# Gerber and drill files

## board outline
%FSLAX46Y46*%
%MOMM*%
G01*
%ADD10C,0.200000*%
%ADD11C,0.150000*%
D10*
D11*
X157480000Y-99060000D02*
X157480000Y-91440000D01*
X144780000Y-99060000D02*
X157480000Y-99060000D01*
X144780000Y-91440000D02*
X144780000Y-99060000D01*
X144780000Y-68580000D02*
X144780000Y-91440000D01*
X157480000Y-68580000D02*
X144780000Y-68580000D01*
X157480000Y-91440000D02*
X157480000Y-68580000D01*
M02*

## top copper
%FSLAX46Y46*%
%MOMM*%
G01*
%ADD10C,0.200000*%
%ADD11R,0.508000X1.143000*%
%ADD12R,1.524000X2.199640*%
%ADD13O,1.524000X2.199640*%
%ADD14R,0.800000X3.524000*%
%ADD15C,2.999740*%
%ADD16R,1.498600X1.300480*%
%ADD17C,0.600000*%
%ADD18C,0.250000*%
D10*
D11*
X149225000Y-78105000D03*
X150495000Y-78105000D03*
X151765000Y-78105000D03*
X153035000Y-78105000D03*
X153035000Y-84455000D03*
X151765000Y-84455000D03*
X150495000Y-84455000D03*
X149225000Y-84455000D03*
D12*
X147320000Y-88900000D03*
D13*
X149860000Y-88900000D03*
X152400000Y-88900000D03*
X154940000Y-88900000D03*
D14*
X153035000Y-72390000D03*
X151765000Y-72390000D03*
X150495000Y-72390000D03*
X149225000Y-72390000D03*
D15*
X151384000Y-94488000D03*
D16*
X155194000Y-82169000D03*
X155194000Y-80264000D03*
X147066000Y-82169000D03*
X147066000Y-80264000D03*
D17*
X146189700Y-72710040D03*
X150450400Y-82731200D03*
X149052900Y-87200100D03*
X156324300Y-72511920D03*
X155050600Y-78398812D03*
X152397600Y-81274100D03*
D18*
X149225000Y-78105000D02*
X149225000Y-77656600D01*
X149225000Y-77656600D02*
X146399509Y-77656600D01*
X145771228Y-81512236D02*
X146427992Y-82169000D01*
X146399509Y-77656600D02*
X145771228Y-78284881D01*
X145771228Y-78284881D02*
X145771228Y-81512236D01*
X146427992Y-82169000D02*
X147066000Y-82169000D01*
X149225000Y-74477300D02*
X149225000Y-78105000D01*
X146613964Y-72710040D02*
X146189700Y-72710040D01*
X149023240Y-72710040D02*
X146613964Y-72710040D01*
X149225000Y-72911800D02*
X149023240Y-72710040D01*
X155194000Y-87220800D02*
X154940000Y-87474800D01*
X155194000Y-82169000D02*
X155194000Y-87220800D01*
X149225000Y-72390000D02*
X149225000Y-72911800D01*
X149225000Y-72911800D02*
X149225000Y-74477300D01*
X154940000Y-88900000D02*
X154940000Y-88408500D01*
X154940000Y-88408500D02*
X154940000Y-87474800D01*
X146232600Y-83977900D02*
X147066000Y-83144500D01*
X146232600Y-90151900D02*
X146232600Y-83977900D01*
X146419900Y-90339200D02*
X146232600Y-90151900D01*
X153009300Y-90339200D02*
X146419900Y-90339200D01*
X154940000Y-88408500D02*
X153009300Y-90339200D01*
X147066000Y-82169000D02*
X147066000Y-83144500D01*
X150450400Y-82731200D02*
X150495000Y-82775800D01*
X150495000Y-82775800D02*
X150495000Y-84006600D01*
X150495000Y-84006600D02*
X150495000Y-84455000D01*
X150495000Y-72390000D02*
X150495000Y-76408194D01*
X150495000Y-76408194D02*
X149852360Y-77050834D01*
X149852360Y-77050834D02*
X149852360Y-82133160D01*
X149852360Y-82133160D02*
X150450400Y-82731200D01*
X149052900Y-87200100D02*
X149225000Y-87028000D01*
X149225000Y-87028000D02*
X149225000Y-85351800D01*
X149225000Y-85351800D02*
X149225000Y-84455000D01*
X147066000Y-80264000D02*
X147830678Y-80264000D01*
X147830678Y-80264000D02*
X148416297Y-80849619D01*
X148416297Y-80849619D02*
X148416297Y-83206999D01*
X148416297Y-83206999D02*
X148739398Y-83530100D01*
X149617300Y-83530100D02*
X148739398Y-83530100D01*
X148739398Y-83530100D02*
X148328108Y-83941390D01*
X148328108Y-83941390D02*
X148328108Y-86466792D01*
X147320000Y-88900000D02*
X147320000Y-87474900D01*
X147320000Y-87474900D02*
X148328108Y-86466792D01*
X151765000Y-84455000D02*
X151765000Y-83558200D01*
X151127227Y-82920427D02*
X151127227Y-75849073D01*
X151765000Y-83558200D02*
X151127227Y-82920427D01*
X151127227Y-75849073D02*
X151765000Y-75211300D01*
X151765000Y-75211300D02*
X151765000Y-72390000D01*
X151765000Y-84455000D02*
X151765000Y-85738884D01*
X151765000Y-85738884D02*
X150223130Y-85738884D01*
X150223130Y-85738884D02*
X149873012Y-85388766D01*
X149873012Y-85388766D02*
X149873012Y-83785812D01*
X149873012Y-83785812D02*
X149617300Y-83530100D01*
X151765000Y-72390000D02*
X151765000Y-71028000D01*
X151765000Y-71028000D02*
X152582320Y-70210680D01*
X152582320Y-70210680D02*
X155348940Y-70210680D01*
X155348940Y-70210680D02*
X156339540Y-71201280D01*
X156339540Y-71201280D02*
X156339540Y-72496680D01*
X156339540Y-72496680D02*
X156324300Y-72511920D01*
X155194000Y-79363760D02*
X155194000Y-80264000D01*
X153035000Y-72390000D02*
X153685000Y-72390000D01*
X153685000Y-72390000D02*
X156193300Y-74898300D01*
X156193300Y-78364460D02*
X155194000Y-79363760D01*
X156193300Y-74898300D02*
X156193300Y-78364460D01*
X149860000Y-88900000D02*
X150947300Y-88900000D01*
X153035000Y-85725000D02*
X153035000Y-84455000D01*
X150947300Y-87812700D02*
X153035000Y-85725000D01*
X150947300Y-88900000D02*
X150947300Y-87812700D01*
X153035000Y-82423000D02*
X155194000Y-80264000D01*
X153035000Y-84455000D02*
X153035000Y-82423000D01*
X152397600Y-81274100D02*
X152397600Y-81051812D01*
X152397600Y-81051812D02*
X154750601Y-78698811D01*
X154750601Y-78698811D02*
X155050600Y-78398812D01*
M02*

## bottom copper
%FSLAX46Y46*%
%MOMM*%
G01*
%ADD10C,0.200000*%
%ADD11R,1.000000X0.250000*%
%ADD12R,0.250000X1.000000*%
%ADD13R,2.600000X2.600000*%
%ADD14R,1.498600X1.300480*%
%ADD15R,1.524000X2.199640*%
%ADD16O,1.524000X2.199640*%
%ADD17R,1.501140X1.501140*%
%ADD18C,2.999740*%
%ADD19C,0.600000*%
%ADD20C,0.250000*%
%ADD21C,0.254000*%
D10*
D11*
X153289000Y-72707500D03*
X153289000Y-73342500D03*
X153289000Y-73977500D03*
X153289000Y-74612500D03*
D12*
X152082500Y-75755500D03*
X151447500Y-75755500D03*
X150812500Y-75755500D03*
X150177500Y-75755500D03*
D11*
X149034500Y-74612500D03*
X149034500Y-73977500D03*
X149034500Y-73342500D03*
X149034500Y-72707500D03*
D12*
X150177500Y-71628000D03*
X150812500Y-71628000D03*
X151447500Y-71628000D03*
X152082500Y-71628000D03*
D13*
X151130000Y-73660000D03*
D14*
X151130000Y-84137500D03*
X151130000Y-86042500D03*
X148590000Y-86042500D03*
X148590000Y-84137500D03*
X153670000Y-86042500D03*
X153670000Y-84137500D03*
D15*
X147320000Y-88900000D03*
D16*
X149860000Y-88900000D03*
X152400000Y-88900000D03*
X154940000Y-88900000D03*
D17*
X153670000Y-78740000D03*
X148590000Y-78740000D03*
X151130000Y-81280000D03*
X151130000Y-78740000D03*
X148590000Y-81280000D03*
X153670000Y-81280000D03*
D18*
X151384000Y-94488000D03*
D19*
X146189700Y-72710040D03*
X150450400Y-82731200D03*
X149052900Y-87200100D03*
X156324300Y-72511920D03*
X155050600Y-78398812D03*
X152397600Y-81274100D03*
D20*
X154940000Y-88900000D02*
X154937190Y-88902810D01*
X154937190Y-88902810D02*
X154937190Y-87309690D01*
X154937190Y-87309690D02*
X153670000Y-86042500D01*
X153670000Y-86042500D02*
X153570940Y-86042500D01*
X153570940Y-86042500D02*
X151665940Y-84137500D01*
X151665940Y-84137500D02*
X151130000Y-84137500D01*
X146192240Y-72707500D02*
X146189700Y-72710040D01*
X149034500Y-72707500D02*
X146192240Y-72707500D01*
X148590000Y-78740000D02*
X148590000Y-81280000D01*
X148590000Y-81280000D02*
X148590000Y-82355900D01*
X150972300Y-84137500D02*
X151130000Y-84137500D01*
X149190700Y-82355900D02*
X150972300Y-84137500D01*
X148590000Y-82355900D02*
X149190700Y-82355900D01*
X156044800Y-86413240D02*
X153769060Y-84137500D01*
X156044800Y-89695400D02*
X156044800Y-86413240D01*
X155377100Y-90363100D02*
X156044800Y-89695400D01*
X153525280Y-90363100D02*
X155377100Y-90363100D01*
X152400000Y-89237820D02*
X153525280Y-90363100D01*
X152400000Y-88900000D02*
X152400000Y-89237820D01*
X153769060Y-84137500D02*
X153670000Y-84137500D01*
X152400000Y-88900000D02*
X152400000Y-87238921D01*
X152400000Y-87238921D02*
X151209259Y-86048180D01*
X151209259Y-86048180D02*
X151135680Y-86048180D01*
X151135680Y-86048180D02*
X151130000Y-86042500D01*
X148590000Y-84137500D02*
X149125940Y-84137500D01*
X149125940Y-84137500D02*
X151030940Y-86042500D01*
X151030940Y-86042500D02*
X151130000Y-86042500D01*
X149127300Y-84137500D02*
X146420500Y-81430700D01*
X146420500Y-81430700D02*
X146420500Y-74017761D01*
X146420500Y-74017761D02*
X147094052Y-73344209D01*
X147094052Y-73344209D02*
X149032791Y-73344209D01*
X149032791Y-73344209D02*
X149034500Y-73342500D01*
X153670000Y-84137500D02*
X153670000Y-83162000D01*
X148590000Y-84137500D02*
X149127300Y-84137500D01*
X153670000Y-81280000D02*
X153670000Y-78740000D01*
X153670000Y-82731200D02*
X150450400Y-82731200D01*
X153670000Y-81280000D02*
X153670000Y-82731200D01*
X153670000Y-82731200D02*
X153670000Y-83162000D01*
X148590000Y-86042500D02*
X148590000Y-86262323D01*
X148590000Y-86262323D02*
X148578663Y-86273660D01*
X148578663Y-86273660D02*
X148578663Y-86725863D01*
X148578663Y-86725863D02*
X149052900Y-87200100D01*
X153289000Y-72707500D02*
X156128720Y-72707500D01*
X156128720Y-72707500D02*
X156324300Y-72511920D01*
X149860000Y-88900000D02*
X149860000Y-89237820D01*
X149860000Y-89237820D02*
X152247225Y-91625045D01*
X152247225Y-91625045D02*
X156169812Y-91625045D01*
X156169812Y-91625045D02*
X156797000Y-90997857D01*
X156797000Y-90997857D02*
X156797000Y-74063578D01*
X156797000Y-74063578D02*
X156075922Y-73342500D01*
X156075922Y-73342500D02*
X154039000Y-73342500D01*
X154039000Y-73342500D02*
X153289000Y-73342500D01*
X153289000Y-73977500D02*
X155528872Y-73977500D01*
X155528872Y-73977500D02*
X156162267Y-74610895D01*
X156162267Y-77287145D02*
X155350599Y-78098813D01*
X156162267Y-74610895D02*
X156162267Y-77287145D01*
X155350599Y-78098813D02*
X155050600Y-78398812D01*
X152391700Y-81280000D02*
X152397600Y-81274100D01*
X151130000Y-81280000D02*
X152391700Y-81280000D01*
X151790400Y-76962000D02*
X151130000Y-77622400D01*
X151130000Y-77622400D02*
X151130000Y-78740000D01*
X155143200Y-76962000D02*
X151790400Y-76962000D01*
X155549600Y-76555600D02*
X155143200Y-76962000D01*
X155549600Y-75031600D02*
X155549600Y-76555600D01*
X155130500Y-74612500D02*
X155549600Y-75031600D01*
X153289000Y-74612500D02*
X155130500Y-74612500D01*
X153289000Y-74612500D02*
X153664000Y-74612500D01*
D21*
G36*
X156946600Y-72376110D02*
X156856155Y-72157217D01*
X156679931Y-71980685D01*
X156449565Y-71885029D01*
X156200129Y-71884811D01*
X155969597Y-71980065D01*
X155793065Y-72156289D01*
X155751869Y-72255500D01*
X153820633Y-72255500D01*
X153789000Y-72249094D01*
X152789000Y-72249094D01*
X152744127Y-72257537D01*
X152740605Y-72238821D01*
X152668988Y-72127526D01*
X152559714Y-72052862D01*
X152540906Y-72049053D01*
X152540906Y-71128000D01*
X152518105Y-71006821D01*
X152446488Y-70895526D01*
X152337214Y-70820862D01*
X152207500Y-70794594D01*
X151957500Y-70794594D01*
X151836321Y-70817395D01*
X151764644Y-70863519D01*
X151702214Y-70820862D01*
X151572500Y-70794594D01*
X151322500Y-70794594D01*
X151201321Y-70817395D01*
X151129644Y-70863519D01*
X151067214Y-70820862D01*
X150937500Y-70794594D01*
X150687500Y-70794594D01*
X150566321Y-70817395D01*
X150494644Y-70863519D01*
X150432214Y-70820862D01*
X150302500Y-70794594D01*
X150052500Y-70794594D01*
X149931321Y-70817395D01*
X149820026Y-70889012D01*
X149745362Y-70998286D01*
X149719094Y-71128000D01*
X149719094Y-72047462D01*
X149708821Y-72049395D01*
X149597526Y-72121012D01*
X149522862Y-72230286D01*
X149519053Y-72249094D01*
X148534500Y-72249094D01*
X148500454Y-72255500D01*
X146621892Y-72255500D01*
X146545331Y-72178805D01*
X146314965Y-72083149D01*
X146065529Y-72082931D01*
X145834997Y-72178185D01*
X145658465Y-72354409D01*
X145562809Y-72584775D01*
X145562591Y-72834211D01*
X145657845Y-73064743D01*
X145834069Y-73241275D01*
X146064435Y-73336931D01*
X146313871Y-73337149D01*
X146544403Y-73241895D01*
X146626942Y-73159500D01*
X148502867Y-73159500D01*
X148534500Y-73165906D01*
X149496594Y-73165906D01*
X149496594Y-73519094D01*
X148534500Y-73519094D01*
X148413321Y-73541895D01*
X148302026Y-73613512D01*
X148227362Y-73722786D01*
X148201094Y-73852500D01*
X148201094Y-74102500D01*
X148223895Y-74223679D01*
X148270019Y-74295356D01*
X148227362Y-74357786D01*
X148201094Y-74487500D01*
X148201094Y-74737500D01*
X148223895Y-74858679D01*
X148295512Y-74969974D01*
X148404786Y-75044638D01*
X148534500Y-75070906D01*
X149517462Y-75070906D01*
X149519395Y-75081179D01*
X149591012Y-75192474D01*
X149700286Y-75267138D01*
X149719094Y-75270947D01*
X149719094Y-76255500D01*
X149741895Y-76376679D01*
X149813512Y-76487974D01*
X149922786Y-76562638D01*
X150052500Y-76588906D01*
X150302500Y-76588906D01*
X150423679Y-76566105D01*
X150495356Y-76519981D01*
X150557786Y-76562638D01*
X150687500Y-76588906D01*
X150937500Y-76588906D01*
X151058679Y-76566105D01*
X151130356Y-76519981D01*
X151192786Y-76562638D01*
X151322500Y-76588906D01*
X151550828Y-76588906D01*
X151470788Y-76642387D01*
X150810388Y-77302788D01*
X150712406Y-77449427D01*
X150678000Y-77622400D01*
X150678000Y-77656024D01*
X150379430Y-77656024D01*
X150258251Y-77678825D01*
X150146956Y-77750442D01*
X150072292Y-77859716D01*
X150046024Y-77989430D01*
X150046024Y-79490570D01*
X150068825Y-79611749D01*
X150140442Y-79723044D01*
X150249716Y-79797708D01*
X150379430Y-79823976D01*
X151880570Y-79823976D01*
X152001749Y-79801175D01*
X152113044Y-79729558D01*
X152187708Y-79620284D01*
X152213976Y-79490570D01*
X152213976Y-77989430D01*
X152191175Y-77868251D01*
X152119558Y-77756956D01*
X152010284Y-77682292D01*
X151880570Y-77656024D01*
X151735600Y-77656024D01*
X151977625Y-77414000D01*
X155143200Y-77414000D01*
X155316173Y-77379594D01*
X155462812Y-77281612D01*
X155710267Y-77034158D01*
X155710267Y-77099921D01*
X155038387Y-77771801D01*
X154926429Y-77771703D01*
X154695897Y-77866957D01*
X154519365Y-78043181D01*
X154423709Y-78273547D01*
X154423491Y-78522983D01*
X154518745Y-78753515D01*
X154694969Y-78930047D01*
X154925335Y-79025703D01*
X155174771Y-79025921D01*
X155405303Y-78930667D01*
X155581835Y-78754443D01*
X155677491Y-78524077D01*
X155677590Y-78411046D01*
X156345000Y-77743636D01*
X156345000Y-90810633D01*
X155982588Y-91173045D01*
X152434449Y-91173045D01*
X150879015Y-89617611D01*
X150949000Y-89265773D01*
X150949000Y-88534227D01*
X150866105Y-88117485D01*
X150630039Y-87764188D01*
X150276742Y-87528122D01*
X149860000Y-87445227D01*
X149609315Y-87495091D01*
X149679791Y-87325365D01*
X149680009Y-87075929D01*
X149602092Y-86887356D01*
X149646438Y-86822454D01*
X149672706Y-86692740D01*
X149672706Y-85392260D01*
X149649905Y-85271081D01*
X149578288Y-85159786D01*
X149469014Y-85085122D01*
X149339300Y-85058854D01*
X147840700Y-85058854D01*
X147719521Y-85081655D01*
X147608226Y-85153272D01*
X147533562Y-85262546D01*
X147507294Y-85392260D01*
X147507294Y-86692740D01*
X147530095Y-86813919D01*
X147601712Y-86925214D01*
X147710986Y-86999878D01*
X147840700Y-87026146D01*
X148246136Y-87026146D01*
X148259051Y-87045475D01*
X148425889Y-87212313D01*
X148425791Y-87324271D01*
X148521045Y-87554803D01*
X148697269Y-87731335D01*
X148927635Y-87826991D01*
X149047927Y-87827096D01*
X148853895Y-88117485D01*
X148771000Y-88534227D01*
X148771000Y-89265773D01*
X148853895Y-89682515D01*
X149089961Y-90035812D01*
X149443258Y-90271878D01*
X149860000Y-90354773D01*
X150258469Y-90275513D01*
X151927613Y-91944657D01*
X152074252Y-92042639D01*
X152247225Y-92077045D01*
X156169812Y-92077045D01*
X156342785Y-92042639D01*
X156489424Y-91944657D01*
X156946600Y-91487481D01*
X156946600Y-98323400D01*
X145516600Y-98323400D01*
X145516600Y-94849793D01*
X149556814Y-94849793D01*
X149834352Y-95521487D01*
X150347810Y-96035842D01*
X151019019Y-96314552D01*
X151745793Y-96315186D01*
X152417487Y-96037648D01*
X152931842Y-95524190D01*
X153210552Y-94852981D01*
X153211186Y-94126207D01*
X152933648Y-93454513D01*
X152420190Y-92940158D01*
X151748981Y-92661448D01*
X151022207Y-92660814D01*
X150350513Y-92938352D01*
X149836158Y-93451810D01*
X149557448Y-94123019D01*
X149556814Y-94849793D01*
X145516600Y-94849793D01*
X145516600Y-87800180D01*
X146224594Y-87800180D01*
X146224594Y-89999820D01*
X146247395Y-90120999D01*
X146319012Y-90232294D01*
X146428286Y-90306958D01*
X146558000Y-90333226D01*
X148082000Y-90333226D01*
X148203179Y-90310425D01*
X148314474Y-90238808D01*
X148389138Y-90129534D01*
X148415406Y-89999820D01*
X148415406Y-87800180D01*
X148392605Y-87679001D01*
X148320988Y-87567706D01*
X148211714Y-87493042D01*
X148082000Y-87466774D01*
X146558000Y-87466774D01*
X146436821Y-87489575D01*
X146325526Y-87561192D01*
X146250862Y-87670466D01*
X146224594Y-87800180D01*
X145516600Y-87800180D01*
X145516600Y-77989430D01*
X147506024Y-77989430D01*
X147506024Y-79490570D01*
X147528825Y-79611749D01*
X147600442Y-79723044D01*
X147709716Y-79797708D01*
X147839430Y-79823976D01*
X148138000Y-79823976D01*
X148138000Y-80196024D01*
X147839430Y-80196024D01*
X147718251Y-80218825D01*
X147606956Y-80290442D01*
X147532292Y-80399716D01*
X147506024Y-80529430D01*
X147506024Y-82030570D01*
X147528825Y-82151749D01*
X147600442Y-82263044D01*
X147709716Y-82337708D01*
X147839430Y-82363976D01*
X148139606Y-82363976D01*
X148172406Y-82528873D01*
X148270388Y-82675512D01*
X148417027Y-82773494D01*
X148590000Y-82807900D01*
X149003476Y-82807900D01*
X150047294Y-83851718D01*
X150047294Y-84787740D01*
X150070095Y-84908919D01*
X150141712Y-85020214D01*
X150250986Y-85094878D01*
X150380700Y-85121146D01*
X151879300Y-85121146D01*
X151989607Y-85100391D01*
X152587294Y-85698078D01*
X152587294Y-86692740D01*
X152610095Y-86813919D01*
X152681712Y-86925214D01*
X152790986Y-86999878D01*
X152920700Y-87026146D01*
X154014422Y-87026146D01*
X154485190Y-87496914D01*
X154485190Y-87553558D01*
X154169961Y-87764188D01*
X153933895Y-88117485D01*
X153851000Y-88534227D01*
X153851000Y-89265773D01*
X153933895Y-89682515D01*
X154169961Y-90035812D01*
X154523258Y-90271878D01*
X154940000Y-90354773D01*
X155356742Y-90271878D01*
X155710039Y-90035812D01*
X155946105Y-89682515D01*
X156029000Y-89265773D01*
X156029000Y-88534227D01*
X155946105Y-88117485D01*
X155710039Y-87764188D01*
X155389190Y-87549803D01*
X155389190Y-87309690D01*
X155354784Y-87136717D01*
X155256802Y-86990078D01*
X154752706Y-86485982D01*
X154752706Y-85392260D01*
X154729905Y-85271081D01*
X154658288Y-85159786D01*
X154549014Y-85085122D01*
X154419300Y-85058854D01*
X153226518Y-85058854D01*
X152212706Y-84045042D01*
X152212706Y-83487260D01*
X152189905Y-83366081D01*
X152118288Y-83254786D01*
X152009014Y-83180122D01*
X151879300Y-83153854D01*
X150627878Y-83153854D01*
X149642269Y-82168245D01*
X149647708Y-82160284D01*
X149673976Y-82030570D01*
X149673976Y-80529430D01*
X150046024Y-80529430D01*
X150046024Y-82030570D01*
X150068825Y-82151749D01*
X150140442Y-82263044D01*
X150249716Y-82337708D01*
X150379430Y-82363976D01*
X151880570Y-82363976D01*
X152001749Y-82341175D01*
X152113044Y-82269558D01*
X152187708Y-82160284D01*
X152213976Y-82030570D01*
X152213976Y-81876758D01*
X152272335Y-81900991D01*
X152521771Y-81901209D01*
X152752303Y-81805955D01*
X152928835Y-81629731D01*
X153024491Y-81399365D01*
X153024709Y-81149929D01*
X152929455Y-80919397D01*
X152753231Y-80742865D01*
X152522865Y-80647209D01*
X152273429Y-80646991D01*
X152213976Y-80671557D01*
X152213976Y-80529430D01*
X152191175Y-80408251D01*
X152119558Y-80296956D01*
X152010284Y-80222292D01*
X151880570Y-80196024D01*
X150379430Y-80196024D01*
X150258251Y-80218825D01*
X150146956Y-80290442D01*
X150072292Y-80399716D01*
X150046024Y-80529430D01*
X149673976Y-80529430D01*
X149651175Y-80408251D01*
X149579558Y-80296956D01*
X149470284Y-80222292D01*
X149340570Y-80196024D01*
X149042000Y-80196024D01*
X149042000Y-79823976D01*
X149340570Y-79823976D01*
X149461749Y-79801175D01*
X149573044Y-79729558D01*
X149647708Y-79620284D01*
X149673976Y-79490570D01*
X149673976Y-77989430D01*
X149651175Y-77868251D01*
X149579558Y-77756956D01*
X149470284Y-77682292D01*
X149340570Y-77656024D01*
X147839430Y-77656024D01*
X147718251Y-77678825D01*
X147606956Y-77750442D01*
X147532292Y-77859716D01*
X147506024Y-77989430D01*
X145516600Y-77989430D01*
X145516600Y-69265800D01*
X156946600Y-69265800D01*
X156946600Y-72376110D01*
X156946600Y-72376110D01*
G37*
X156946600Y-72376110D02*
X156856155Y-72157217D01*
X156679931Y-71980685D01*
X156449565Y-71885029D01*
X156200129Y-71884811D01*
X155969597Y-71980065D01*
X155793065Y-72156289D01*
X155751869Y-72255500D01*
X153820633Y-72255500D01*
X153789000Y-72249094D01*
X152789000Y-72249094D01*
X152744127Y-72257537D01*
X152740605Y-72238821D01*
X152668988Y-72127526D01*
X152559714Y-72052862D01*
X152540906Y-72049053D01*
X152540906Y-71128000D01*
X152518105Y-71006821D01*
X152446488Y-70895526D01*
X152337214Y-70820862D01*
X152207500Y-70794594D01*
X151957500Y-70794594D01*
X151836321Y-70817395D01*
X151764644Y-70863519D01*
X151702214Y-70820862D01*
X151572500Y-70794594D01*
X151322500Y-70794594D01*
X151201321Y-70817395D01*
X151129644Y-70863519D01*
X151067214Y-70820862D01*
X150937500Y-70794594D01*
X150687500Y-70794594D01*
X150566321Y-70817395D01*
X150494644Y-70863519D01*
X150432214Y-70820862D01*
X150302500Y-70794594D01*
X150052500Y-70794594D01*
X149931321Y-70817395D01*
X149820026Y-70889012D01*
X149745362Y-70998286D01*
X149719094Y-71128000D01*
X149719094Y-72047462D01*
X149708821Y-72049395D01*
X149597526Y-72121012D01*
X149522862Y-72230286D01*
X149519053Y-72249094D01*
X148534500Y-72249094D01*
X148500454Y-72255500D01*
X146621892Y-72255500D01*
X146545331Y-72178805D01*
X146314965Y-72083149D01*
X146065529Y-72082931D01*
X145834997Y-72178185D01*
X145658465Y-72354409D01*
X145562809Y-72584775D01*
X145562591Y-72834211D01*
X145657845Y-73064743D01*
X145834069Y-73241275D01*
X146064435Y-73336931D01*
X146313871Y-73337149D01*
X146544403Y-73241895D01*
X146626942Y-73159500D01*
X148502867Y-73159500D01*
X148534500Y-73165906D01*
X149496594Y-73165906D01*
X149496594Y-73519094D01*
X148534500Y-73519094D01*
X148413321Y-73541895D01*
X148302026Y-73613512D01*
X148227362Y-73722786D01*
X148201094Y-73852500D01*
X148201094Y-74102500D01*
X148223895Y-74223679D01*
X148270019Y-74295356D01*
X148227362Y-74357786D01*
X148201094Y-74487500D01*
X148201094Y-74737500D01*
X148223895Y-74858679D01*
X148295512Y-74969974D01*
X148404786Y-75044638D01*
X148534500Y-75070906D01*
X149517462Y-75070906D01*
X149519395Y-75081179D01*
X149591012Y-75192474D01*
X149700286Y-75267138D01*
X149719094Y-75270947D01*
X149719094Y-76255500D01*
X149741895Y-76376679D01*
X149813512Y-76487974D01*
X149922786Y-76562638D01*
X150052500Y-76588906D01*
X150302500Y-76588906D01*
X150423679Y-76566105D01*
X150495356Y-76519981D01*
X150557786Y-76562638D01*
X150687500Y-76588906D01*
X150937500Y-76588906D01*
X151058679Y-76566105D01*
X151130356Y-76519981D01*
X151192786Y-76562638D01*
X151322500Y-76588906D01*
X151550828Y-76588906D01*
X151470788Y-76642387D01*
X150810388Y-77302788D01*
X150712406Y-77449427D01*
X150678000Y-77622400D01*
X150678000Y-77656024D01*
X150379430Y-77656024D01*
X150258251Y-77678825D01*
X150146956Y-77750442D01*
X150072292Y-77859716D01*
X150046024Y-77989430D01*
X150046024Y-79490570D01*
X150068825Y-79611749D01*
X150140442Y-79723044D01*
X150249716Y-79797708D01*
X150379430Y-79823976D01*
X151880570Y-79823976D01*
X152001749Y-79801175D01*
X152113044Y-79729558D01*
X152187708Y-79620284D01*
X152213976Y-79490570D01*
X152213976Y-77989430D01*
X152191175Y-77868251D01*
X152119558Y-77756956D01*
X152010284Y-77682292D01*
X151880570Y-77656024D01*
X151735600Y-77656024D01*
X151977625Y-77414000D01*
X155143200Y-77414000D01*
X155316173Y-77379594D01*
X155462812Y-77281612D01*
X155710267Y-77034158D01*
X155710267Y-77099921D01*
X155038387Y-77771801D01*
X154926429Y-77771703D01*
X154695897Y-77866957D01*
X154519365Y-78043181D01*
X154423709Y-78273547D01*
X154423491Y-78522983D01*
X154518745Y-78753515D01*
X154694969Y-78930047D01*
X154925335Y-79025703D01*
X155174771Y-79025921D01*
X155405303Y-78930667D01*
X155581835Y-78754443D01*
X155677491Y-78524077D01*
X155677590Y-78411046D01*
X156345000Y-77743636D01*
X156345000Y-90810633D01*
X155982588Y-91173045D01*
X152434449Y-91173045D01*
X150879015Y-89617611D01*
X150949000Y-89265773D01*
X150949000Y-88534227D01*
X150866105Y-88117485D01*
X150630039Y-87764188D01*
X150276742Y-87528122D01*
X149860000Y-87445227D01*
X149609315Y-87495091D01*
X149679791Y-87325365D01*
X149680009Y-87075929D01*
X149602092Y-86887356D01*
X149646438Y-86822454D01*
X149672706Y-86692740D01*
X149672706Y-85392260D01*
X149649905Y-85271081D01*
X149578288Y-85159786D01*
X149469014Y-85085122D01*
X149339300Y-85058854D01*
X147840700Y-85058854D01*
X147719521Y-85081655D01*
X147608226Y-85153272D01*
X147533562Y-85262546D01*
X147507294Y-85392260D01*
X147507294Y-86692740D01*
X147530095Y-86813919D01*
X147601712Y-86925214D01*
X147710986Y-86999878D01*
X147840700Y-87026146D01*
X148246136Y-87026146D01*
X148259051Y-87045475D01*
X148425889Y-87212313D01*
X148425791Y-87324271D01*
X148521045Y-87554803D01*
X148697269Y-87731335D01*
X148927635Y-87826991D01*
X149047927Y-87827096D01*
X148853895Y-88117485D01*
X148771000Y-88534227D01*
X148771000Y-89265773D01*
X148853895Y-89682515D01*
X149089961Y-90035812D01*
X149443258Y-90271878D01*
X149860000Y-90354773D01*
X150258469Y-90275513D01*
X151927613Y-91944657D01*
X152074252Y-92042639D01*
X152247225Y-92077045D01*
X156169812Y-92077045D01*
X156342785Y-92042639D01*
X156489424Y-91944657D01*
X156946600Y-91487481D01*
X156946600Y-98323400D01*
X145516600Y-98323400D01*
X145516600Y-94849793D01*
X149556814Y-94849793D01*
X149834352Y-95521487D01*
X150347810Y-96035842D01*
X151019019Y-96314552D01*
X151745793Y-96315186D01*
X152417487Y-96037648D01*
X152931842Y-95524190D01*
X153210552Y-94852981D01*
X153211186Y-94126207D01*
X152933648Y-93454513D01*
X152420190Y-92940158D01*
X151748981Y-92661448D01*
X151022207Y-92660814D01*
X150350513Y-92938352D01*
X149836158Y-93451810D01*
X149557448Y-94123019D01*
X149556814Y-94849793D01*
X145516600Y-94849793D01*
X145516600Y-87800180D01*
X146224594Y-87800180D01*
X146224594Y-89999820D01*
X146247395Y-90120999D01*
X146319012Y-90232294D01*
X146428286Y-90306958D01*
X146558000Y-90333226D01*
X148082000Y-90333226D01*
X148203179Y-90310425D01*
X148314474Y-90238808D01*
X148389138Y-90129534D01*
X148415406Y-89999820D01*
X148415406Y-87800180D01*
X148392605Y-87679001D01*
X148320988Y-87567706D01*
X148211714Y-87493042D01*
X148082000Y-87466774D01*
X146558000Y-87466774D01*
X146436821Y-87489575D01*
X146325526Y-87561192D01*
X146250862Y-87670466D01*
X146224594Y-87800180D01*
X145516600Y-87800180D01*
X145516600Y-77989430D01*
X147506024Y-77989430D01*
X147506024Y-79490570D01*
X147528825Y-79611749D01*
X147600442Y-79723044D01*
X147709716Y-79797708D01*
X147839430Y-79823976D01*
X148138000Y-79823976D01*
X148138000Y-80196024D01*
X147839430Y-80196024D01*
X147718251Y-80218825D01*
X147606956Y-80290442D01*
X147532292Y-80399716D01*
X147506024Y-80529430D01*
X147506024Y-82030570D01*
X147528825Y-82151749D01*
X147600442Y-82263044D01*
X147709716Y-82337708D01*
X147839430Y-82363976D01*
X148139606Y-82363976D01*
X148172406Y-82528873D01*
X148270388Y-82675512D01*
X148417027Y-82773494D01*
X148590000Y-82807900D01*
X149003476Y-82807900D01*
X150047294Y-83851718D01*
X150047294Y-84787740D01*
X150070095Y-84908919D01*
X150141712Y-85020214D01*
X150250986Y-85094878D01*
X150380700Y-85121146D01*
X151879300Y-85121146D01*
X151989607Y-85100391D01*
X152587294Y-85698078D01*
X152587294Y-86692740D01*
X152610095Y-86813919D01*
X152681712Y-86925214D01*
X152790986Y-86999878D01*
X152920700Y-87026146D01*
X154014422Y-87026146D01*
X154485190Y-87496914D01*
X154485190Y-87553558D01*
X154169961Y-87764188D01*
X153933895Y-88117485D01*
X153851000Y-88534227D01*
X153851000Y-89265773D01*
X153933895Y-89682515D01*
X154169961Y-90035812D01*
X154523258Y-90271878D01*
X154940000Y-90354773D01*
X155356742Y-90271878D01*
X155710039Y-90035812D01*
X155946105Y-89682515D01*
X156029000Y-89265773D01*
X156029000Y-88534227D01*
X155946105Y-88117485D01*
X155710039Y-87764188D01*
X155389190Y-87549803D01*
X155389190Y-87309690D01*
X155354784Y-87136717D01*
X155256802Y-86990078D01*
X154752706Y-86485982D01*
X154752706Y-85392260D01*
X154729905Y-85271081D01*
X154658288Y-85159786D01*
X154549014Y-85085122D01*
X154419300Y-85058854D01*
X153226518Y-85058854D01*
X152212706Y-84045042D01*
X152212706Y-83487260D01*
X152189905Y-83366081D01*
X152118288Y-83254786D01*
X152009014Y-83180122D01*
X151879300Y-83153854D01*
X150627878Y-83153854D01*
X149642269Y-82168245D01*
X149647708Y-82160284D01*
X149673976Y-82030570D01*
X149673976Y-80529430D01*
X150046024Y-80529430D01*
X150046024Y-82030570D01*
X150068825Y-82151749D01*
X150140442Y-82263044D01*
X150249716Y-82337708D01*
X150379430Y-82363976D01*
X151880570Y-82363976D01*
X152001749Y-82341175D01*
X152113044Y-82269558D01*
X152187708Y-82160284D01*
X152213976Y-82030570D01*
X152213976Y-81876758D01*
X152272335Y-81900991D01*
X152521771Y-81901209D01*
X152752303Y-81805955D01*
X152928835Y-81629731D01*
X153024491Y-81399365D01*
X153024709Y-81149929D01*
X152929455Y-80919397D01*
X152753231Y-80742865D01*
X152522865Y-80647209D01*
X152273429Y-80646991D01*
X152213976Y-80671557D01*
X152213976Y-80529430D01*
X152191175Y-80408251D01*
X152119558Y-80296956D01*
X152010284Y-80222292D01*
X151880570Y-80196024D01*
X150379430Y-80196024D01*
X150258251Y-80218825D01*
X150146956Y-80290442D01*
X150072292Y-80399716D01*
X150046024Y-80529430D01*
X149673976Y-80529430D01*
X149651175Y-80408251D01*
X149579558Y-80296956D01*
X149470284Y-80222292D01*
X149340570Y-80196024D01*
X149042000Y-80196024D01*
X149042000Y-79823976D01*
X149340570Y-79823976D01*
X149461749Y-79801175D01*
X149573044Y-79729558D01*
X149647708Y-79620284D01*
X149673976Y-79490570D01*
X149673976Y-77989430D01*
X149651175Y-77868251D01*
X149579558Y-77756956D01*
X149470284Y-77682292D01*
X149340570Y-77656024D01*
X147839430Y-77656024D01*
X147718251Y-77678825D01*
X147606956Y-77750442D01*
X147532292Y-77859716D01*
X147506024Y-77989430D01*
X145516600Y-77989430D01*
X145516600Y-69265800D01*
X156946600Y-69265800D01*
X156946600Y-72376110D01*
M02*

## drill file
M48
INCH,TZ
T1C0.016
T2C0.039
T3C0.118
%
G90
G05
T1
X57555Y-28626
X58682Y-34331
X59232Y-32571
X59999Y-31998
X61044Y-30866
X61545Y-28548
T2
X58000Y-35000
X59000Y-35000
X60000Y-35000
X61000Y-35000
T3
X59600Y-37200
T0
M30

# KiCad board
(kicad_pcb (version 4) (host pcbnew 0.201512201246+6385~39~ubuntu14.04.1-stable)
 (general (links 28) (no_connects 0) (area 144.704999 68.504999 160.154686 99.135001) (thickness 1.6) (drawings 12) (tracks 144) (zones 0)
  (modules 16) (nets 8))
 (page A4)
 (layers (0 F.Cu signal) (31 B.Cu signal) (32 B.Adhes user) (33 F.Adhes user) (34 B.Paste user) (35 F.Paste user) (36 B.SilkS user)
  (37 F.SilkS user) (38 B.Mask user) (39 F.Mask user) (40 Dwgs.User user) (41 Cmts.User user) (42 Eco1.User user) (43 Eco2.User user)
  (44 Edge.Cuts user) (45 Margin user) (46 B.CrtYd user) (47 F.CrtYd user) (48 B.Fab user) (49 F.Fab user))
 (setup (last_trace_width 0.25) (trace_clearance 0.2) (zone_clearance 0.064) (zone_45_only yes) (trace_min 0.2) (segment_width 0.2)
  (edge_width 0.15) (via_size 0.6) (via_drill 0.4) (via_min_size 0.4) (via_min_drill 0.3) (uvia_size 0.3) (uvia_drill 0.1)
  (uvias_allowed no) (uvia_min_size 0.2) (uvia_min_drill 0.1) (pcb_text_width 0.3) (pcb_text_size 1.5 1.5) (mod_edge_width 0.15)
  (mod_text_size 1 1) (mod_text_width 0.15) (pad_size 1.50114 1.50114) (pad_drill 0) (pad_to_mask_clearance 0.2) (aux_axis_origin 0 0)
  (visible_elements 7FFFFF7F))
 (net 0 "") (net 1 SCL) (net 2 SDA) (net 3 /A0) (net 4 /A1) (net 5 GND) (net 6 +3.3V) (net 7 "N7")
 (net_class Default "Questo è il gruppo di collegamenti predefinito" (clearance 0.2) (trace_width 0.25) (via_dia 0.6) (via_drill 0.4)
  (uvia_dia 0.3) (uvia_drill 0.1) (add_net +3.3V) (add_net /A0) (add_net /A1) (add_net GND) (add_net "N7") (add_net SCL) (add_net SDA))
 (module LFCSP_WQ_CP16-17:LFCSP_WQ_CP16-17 (layer B.Cu) (at 151.13 73.66 180)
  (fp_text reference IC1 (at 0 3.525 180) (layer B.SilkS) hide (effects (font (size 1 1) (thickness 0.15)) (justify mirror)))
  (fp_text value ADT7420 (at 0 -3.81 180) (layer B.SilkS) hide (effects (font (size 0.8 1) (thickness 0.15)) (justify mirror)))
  (pad 1 smd rect (at -2.159 0.9525 180) (size 1 0.25) (layers B.Cu B.Paste B.Mask) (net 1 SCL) (solder_mask_margin 0.07))
  (pad 2 smd rect (at -2.159 0.3175 180) (size 1 0.25) (layers B.Cu B.Paste B.Mask) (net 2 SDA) (solder_mask_margin 0.07))
  (pad 3 smd rect (at -2.159 -0.3175 180) (size 1 0.25) (layers B.Cu B.Paste B.Mask) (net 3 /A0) (solder_mask_margin 0.07))
  (pad 4 smd rect (at -2.159 -0.9525 180) (size 1 0.25) (layers B.Cu B.Paste B.Mask) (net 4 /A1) (solder_mask_margin 0.07))
  (pad 5 smd rect (at -0.9525 -2.0955 90) (size 1 0.25) (layers B.Cu B.Paste B.Mask) (solder_mask_margin 0.07))
  (pad 6 smd rect (at -0.3175 -2.0955 90) (size 1 0.25) (layers B.Cu B.Paste B.Mask) (solder_mask_margin 0.07))
  (pad 7 smd rect (at 0.3175 -2.0955 90) (size 1 0.25) (layers B.Cu B.Paste B.Mask) (solder_mask_margin 0.07))
  (pad 8 smd rect (at 0.9525 -2.0955 90) (size 1 0.25) (layers B.Cu B.Paste B.Mask) (solder_mask_margin 0.07))
  (pad 9 smd rect (at 2.0955 -0.9525 270) (size 0.25 1) (layers B.Cu B.Paste B.Mask) (solder_mask_margin 0.07))
  (pad 10 smd rect (at 2.0955 -0.3175 270) (size 0.25 1) (layers B.Cu B.Paste B.Mask) (solder_mask_margin 0.07))
  (pad 11 smd rect (at 2.0955 0.3175 270) (size 0.25 1) (layers B.Cu B.Paste B.Mask) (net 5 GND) (solder_mask_margin 0.07))
  (pad 12 smd rect (at 2.0955 0.9525 270) (size 0.25 1) (layers B.Cu B.Paste B.Mask) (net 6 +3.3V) (solder_mask_margin 0.07))
  (pad 13 smd rect (at 0.9525 2.032 180) (size 0.25 1) (layers B.Cu B.Paste B.Mask) (solder_mask_margin 0.07))
  (pad 14 smd rect (at 0.3175 2.032 180) (size 0.25 1) (layers B.Cu B.Paste B.Mask) (solder_mask_margin 0.07))
  (pad 15 smd rect (at -0.3175 2.032 180) (size 0.25 1) (layers B.Cu B.Paste B.Mask) (solder_mask_margin 0.07))
  (pad 16 smd rect (at -0.9525 2.032 180) (size 0.25 1) (layers B.Cu B.Paste B.Mask) (solder_mask_margin 0.07))
  (pad 17 smd rect (at 0 0 180) (size 2.6 2.6) (layers B.Cu B.Paste B.Mask)))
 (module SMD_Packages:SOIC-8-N (layer F.Cu) (at 151.13 81.28)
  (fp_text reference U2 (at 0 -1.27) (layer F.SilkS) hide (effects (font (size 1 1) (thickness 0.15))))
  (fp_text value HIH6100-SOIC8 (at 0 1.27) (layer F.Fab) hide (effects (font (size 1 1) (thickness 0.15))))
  (pad 8 smd rect (at -1.905 -3.175) (size 0.508 1.143) (layers F.Cu F.Paste F.Mask) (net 6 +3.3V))
  (pad 7 smd rect (at -0.635 -3.175) (size 0.508 1.143) (layers F.Cu F.Paste F.Mask))
  (pad 6 smd rect (at 0.635 -3.175) (size 0.508 1.143) (layers F.Cu F.Paste F.Mask))
  (pad 5 smd rect (at 1.905 -3.175) (size 0.508 1.143) (layers F.Cu F.Paste F.Mask))
  (pad 4 smd rect (at 1.905 3.175) (size 0.508 1.143) (layers F.Cu F.Paste F.Mask) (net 2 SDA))
  (pad 3 smd rect (at 0.635 3.175) (size 0.508 1.143) (layers F.Cu F.Paste F.Mask) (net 1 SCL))
  (pad 2 smd rect (at -0.635 3.175) (size 0.508 1.143) (layers F.Cu F.Paste F.Mask) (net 5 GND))
  (pad 1 smd rect (at -1.905 3.175) (size 0.508 1.143) (layers F.Cu F.Paste F.Mask) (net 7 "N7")))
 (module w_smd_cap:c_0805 (layer B.Cu) (at 151.13 85.09 90)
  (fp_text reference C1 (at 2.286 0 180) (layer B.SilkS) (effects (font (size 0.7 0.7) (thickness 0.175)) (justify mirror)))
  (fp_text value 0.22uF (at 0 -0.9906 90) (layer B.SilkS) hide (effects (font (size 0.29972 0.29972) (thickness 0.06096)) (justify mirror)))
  (pad 1 smd rect (at 0.9525 0 90) (size 1.30048 1.4986) (layers B.Cu B.Paste B.Mask) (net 6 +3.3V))
  (pad 2 smd rect (at -0.9525 0 90) (size 1.30048 1.4986) (layers B.Cu B.Paste B.Mask) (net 5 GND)))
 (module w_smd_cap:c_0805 (layer B.Cu) (at 148.59 85.09 270)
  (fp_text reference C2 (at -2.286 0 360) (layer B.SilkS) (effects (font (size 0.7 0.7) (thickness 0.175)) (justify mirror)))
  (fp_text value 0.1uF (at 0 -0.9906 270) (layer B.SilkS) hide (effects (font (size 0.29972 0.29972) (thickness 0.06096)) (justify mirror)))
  (pad 1 smd rect (at 0.9525 0 270) (size 1.30048 1.4986) (layers B.Cu B.Paste B.Mask) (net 7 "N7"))
  (pad 2 smd rect (at -0.9525 0 270) (size 1.30048 1.4986) (layers B.Cu B.Paste B.Mask) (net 5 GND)))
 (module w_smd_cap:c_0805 (layer B.Cu) (at 153.67 85.09 270)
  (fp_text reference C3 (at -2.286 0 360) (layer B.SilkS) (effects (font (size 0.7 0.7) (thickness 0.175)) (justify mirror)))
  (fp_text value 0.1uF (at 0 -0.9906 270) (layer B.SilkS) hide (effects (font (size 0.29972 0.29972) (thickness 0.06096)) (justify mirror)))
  (pad 1 smd rect (at 0.9525 0 270) (size 1.30048 1.4986) (layers B.Cu B.Paste B.Mask) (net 6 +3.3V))
  (pad 2 smd rect (at -0.9525 0 270) (size 1.30048 1.4986) (layers B.Cu B.Paste B.Mask) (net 5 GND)))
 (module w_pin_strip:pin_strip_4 (layer F.Cu) (at 151.13 88.9)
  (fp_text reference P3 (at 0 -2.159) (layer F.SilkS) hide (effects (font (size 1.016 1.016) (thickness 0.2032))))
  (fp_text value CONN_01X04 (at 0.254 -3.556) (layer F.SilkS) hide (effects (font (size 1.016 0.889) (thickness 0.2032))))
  (pad 1 thru_hole rect (at -3.81 0) (size 1.524 2.19964) (drill 1.00076) (layers *.Cu *.Mask F.SilkS) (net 1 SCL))
  (pad 2 thru_hole oval (at -1.27 0) (size 1.524 2.19964) (drill 1.00076) (layers *.Cu *.Mask F.SilkS) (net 2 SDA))
  (pad 3 thru_hole oval (at 1.27 0) (size 1.524 2.19964) (drill 1.00076) (layers *.Cu *.Mask F.SilkS) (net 5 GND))
  (pad 4 thru_hole oval (at 3.81 0) (size 1.524 2.19964) (drill 1.00076) (layers *.Cu *.Mask F.SilkS) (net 6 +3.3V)))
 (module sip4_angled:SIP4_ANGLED (layer F.Cu) (at 151.13 71.12)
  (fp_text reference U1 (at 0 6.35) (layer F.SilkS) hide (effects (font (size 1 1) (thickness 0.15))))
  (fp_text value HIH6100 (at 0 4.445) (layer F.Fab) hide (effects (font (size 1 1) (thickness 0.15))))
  (pad 4 smd rect (at 1.905 1.27) (size 0.8 3.524) (layers F.Cu F.Paste F.Mask) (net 2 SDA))
  (pad 3 smd rect (at 0.635 1.27) (size 0.8 3.524) (layers F.Cu F.Paste F.Mask) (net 1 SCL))
  (pad 2 smd rect (at -0.635 1.27) (size 0.8 3.524) (layers F.Cu F.Paste F.Mask) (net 5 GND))
  (pad 1 smd rect (at -1.905 1.27) (size 0.8 3.524) (layers F.Cu F.Paste F.Mask) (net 6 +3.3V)))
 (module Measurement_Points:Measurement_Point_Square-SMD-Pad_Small (layer B.Cu) (at 153.67 78.74)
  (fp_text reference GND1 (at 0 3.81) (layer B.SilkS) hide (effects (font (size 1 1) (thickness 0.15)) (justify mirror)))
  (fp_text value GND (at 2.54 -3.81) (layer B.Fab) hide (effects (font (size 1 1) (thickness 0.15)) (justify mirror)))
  (pad 1 smd rect (at 0 0) (size 1.50114 1.50114) (layers B.Cu B.Paste B.Mask) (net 5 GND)))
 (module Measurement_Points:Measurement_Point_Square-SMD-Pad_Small (layer B.Cu) (at 148.59 78.74)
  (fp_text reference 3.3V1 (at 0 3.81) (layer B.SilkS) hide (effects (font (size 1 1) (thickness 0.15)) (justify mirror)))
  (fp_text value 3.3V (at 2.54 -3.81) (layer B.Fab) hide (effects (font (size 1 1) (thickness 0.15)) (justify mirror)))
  (pad 1 smd rect (at 0 0) (size 1.50114 1.50114) (layers B.Cu B.Paste B.Mask) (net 6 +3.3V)))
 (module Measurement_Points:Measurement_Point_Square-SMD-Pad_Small (layer B.Cu) (at 151.13 81.28)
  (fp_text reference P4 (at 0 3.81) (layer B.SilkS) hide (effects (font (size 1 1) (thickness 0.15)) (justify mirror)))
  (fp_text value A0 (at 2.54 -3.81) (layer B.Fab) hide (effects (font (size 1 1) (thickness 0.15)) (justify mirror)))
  (pad 1 smd rect (at 0 0) (size 1.50114 1.50114) (layers B.Cu B.Paste B.Mask) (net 3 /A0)))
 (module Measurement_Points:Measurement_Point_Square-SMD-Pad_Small (layer B.Cu) (at 151.13 78.74)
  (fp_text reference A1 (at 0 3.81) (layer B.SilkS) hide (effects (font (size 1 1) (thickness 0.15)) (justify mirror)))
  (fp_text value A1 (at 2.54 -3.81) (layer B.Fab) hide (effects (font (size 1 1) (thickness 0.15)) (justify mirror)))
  (pad 1 smd rect (at 0 0) (size 1.50114 1.50114) (layers B.Cu B.Paste B.Mask) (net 4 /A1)))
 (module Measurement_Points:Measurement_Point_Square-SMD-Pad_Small (layer F.Cu) (at 148.59 81.28)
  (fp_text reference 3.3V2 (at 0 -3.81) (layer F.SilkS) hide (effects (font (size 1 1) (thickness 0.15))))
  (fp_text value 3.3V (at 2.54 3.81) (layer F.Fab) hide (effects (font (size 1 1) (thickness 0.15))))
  (pad 1 smd rect (at 0 0) (size 1.50114 1.50114) (layers B.Cu B.Paste B.Mask) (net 6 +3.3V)))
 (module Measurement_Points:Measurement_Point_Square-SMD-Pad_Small (layer F.Cu) (at 153.67 81.28)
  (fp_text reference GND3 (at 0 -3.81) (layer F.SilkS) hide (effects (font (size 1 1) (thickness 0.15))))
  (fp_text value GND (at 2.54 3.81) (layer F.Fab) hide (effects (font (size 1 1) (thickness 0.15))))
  (pad 1 smd rect (at 0 0) (size 1.50114 1.50114) (layers B.Cu B.Paste B.Mask) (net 5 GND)))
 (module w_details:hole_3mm (layer F.Cu) (at 151.384 94.488)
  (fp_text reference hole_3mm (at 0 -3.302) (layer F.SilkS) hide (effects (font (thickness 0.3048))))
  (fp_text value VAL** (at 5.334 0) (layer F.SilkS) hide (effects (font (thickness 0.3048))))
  (pad 1 thru_hole circle (at 0 0) (size 2.99974 2.99974) (drill 2.99974) (layers *.Cu F.SilkS)))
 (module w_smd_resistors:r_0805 (layer F.Cu) (at 155.194 81.2165 270)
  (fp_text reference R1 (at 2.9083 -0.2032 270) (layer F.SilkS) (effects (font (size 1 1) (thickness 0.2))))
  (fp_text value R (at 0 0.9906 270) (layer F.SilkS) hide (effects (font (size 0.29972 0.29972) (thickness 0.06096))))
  (pad 1 smd rect (at 0.9525 0 270) (size 1.30048 1.4986) (layers F.Cu F.Paste F.Mask) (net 6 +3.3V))
  (pad 2 smd rect (at -0.9525 0 270) (size 1.30048 1.4986) (layers F.Cu F.Paste F.Mask) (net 2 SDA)))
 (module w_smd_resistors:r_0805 (layer F.Cu) (at 147.066 81.2165 270)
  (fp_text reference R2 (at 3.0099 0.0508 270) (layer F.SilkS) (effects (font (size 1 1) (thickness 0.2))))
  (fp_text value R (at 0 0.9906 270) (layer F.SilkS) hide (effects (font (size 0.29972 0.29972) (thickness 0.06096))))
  (pad 1 smd rect (at 0.9525 0 270) (size 1.30048 1.4986) (layers F.Cu F.Paste F.Mask) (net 6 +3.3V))
  (pad 2 smd rect (at -0.9525 0 270) (size 1.30048 1.4986) (layers F.Cu F.Paste F.Mask) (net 1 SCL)))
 (gr_line (start 157.48 99.06) (end 157.48 91.44) (angle 90) (layer Edge.Cuts) (width 0.15))
 (gr_line (start 144.78 99.06) (end 157.48 99.06) (angle 90) (layer Edge.Cuts) (width 0.15))
 (gr_line (start 144.78 91.44) (end 144.78 99.06) (angle 90) (layer Edge.Cuts) (width 0.15))
 (gr_line (start 144.78 68.58) (end 144.78 91.44) (angle 90) (layer Edge.Cuts) (width 0.15))
 (gr_line (start 157.48 68.58) (end 144.78 68.58) (angle 90) (layer Edge.Cuts) (width 0.15))
 (gr_line (start 157.48 91.44) (end 157.48 68.58) (angle 90) (layer Edge.Cuts) (width 0.15))
 (segment (start 154.94 88.9) (end 154.93719 88.90281) (width 0.25) (layer B.Cu) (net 6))
 (segment (start 154.93719 88.90281) (end 154.93719 87.30969) (width 0.25) (layer B.Cu) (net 6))
 (segment (start 154.93719 87.30969) (end 153.67 86.0425) (width 0.25) (layer B.Cu) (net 6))
 (segment (start 149.225 78.105) (end 149.225 77.6566) (width 0.25) (layer F.Cu) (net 6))
 (segment (start 149.225 77.6566) (end 146.399509 77.6566) (width 0.25) (layer F.Cu) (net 6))
 (segment (start 145.771228 81.512236) (end 146.427992 82.169) (width 0.25) (layer F.Cu) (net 6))
 (segment (start 146.399509 77.6566) (end 145.771228 78.284881) (width 0.25) (layer F.Cu) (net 6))
 (segment (start 145.771228 78.284881) (end 145.771228 81.512236) (width 0.25) (layer F.Cu) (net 6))
 (segment (start 146.427992 82.169) (end 147.066 82.169) (width 0.25) (layer F.Cu) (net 6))
 (segment (start 149.225 74.4773) (end 149.225 78.105) (width 0.25) (layer F.Cu) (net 6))
 (segment (start 153.67 86.0425) (end 153.57094 86.0425) (width 0.25) (layer B.Cu) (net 6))
 (segment (start 153.57094 86.0425) (end 151.66594 84.1375) (width 0.25) (layer B.Cu) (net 6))
 (segment (start 151.66594 84.1375) (end 151.13 84.1375) (width 0.25) (layer B.Cu) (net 6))
 (segment (start 146.613964 72.71004) (end 146.1897 72.71004) (width 0.25) (layer F.Cu) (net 6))
 (segment (start 149.02324 72.71004) (end 146.613964 72.71004) (width 0.25) (layer F.Cu) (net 6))
 (segment (start 149.225 72.9118) (end 149.02324 72.71004) (width 0.25) (layer F.Cu) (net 6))
 (segment (start 146.19224 72.7075) (end 146.1897 72.71004) (width 0.25) (layer B.Cu) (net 6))
 (segment (start 149.0345 72.7075) (end 146.19224 72.7075) (width 0.25) (layer B.Cu) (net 6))
 (via (at 146.1897 72.71004) (size 0.6) (drill 0.4) (layers F.Cu B.Cu) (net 6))
 (segment (start 155.194 87.2208) (end 154.94 87.4748) (width 0.25) (layer F.Cu) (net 6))
 (segment (start 155.194 82.169) (end 155.194 87.2208) (width 0.25) (layer F.Cu) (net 6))
 (segment (start 149.225 72.39) (end 149.225 72.9118) (width 0.25) (layer F.Cu) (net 6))
 (segment (start 149.225 72.9118) (end 149.225 74.4773) (width 0.25) (layer F.Cu) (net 6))
 (segment (start 148.59 78.74) (end 148.59 81.28) (width 0.25) (layer B.Cu) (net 6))
 (segment (start 148.59 81.28) (end 148.59 82.3559) (width 0.25) (layer B.Cu) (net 6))
 (segment (start 150.9723 84.1375) (end 151.13 84.1375) (width 0.25) (layer B.Cu) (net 6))
 (segment (start 149.1907 82.3559) (end 150.9723 84.1375) (width 0.25) (layer B.Cu) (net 6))
 (segment (start 148.59 82.3559) (end 149.1907 82.3559) (width 0.25) (layer B.Cu) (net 6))
 (segment (start 154.94 88.9) (end 154.94 88.4085) (width 0.25) (layer F.Cu) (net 6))
 (segment (start 154.94 88.4085) (end 154.94 87.4748) (width 0.25) (layer F.Cu) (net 6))
 (segment (start 146.2326 83.9779) (end 147.066 83.1445) (width 0.25) (layer F.Cu) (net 6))
 (segment (start 146.2326 90.1519) (end 146.2326 83.9779) (width 0.25) (layer F.Cu) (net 6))
 (segment (start 146.4199 90.3392) (end 146.2326 90.1519) (width 0.25) (layer F.Cu) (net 6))
 (segment (start 153.0093 90.3392) (end 146.4199 90.3392) (width 0.25) (layer F.Cu) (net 6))
 (segment (start 154.94 88.4085) (end 153.0093 90.3392) (width 0.25) (layer F.Cu) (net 6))
 (segment (start 147.066 82.169) (end 147.066 83.1445) (width 0.25) (layer F.Cu) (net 6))
 (segment (start 150.4504 82.7312) (end 150.495 82.7758) (width 0.25) (layer F.Cu) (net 5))
 (segment (start 150.495 82.7758) (end 150.495 84.0066) (width 0.25) (layer F.Cu) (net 5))
 (segment (start 150.495 84.0066) (end 150.495 84.455) (width 0.25) (layer F.Cu) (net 5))
 (segment (start 156.0448 86.41324) (end 153.76906 84.1375) (width 0.25) (layer B.Cu) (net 5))
 (segment (start 156.0448 89.6954) (end 156.0448 86.41324) (width 0.25) (layer B.Cu) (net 5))
 (segment (start 155.3771 90.3631) (end 156.0448 89.6954) (width 0.25) (layer B.Cu) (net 5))
 (segment (start 153.52528 90.3631) (end 155.3771 90.3631) (width 0.25) (layer B.Cu) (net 5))
 (segment (start 152.4 89.23782) (end 153.52528 90.3631) (width 0.25) (layer B.Cu) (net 5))
 (segment (start 152.4 88.9) (end 152.4 89.23782) (width 0.25) (layer B.Cu) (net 5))
 (segment (start 153.76906 84.1375) (end 153.67 84.1375) (width 0.25) (layer B.Cu) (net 5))
 (segment (start 152.4 88.9) (end 152.4 87.238921) (width 0.25) (layer B.Cu) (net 5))
 (segment (start 152.4 87.238921) (end 151.209259 86.04818) (width 0.25) (layer B.Cu) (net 5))
 (segment (start 151.209259 86.04818) (end 151.13568 86.04818) (width 0.25) (layer B.Cu) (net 5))
 (segment (start 151.13568 86.04818) (end 151.13 86.0425) (width 0.25) (layer B.Cu) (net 5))
 (segment (start 150.495 72.39) (end 150.495 76.408194) (width 0.25) (layer F.Cu) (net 5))
 (segment (start 150.495 76.408194) (end 149.85236 77.050834) (width 0.25) (layer F.Cu) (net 5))
 (segment (start 149.85236 77.050834) (end 149.85236 82.13316) (width 0.25) (layer F.Cu) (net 5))
 (segment (start 149.85236 82.13316) (end 150.4504 82.7312) (width 0.25) (layer F.Cu) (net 5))
 (segment (start 148.59 84.1375) (end 149.12594 84.1375) (width 0.25) (layer B.Cu) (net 5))
 (segment (start 149.12594 84.1375) (end 151.03094 86.0425) (width 0.25) (layer B.Cu) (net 5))
 (segment (start 151.03094 86.0425) (end 151.13 86.0425) (width 0.25) (layer B.Cu) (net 5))
 (segment (start 149.1273 84.1375) (end 146.4205 81.4307) (width 0.25) (layer B.Cu) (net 5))
 (segment (start 146.4205 81.4307) (end 146.4205 74.017761) (width 0.25) (layer B.Cu) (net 5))
 (segment (start 146.4205 74.017761) (end 147.094052 73.344209) (width 0.25) (layer B.Cu) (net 5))
 (segment (start 147.094052 73.344209) (end 149.032791 73.344209) (width 0.25) (layer B.Cu) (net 5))
 (segment (start 149.032791 73.344209) (end 149.0345 73.3425) (width 0.25) (layer B.Cu) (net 5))
 (via (at 150.4504 82.7312) (size 0.6) (layers F.Cu B.Cu) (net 5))
 (segment (start 153.67 84.1375) (end 153.67 83.162) (width 0.25) (layer B.Cu) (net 5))
 (segment (start 148.59 84.1375) (end 149.1273 84.1375) (width 0.25) (layer B.Cu) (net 5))
 (segment (start 153.67 81.28) (end 153.67 78.74) (width 0.25) (layer B.Cu) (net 5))
 (segment (start 153.67 82.7312) (end 150.4504 82.7312) (width 0.25) (layer B.Cu) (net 5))
 (segment (start 153.67 81.28) (end 153.67 82.7312) (width 0.25) (layer B.Cu) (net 5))
 (segment (start 153.67 82.7312) (end 153.67 83.162) (width 0.25) (layer B.Cu) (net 5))
 (segment (start 148.59 86.0425) (end 148.59 86.262323) (width 0.25) (layer B.Cu) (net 7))
 (segment (start 148.59 86.262323) (end 148.578663 86.27366) (width 0.25) (layer B.Cu) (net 7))
 (segment (start 148.578663 86.27366) (end 148.578663 86.725863) (width 0.25) (layer B.Cu) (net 7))
 (segment (start 148.578663 86.725863) (end 149.0529 87.2001) (width 0.25) (layer B.Cu) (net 7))
 (segment (start 149.0529 87.2001) (end 149.225 87.028) (width 0.25) (layer F.Cu) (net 7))
 (segment (start 149.225 87.028) (end 149.225 85.3518) (width 0.25) (layer F.Cu) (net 7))
 (segment (start 149.225 85.3518) (end 149.225 84.455) (width 0.25) (layer F.Cu) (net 7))
 (via (at 149.0529 87.2001) (size 0.6) (layers F.Cu B.Cu) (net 7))
 (segment (start 147.066 80.264) (end 147.830678 80.264) (width 0.25) (layer F.Cu) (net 1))
 (segment (start 147.830678 80.264) (end 148.416297 80.849619) (width 0.25) (layer F.Cu) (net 1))
 (segment (start 148.416297 80.849619) (end 148.416297 83.206999) (width 0.25) (layer F.Cu) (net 1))
 (segment (start 148.416297 83.206999) (end 148.739398 83.5301) (width 0.25) (layer F.Cu) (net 1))
 (segment (start 149.6173 83.5301) (end 148.739398 83.5301) (width 0.25) (layer F.Cu) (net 1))
 (segment (start 148.739398 83.5301) (end 148.328108 83.94139) (width 0.25) (layer F.Cu) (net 1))
 (segment (start 148.328108 83.94139) (end 148.328108 86.466792) (width 0.25) (layer F.Cu) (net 1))
 (segment (start 147.32 88.9) (end 147.32 87.4749) (width 0.25) (layer F.Cu) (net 1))
 (segment (start 147.32 87.4749) (end 148.328108 86.466792) (width 0.25) (layer F.Cu) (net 1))
 (segment (start 151.765 84.455) (end 151.765 83.5582) (width 0.25) (layer F.Cu) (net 1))
 (segment (start 151.127227 82.920427) (end 151.127227 75.849073) (width 0.25) (layer F.Cu) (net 1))
 (segment (start 151.765 83.5582) (end 151.127227 82.920427) (width 0.25) (layer F.Cu) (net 1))
 (segment (start 151.127227 75.849073) (end 151.765 75.2113) (width 0.25) (layer F.Cu) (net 1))
 (segment (start 151.765 75.2113) (end 151.765 72.39) (width 0.25) (layer F.Cu) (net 1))
 (segment (start 151.765 84.455) (end 151.765 85.738884) (width 0.25) (layer F.Cu) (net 1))
 (segment (start 151.765 85.738884) (end 150.22313 85.738884) (width 0.25) (layer F.Cu) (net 1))
 (segment (start 150.22313 85.738884) (end 149.873012 85.388766) (width 0.25) (layer F.Cu) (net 1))
 (segment (start 149.873012 85.388766) (end 149.873012 83.785812) (width 0.25) (layer F.Cu) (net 1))
 (segment (start 149.873012 83.785812) (end 149.6173 83.5301) (width 0.25) (layer F.Cu) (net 1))
 (segment (start 151.765 72.39) (end 151.765 71.028) (width 0.25) (layer F.Cu) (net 1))
 (segment (start 151.765 71.028) (end 152.58232 70.21068) (width 0.25) (layer F.Cu) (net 1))
 (segment (start 152.58232 70.21068) (end 155.34894 70.21068) (width 0.25) (layer F.Cu) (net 1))
 (segment (start 155.34894 70.21068) (end 156.33954 71.20128) (width 0.25) (layer F.Cu) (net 1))
 (segment (start 156.33954 71.20128) (end 156.33954 72.49668) (width 0.25) (layer F.Cu) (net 1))
 (segment (start 156.33954 72.49668) (end 156.3243 72.51192) (width 0.25) (layer F.Cu) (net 1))
 (segment (start 153.289 72.7075) (end 156.12872 72.7075) (width 0.25) (layer B.Cu) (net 1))
 (segment (start 156.12872 72.7075) (end 156.3243 72.51192) (width 0.25) (layer B.Cu) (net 1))
 (via (at 156.3243 72.51192) (size 0.6) (drill 0.4) (layers F.Cu B.Cu) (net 1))
 (segment (start 149.86 88.9) (end 149.86 89.23782) (width 0.25) (layer B.Cu) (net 2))
 (segment (start 149.86 89.23782) (end 152.247225 91.625045) (width 0.25) (layer B.Cu) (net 2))
 (segment (start 152.247225 91.625045) (end 156.169812 91.625045) (width 0.25) (layer B.Cu) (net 2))
 (segment (start 156.169812 91.625045) (end 156.797 90.997857) (width 0.25) (layer B.Cu) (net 2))
 (segment (start 156.797 90.997857) (end 156.797 74.063578) (width 0.25) (layer B.Cu) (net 2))
 (segment (start 156.797 74.063578) (end 156.075922 73.3425) (width 0.25) (layer B.Cu) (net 2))
 (segment (start 156.075922 73.3425) (end 154.039 73.3425) (width 0.25) (layer B.Cu) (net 2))
 (segment (start 154.039 73.3425) (end 153.289 73.3425) (width 0.25) (layer B.Cu) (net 2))
 (segment (start 155.194 79.36376) (end 155.194 80.264) (width 0.25) (layer F.Cu) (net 2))
 (segment (start 153.035 72.39) (end 153.685 72.39) (width 0.25) (layer F.Cu) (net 2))
 (segment (start 153.685 72.39) (end 156.1933 74.8983) (width 0.25) (layer F.Cu) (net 2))
 (segment (start 156.1933 78.36446) (end 155.194 79.36376) (width 0.25) (layer F.Cu) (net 2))
 (segment (start 156.1933 74.8983) (end 156.1933 78.36446) (width 0.25) (layer F.Cu) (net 2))
 (segment (start 149.86 88.9) (end 150.9473 88.9) (width 0.25) (layer F.Cu) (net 2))
 (segment (start 153.035 85.725) (end 153.035 84.455) (width 0.25) (layer F.Cu) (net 2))
 (segment (start 150.9473 87.8127) (end 153.035 85.725) (width 0.25) (layer F.Cu) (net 2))
 (segment (start 150.9473 88.9) (end 150.9473 87.8127) (width 0.25) (layer F.Cu) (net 2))
 (segment (start 153.035 82.423) (end 155.194 80.264) (width 0.25) (layer F.Cu) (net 2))
 (segment (start 153.035 84.455) (end 153.035 82.423) (width 0.25) (layer F.Cu) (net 2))
 (segment (start 152.3976 81.2741) (end 152.3976 81.051812) (width 0.25) (layer F.Cu) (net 3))
 (segment (start 152.3976 81.051812) (end 154.750601 78.698811) (width 0.25) (layer F.Cu) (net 3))
 (segment (start 154.750601 78.698811) (end 155.0506 78.398812) (width 0.25) (layer F.Cu) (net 3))
 (segment (start 153.289 73.9775) (end 155.528872 73.9775) (width 0.25) (layer B.Cu) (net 3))
 (segment (start 155.528872 73.9775) (end 156.162267 74.610895) (width 0.25) (layer B.Cu) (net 3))
 (segment (start 156.162267 77.287145) (end 155.350599 78.098813) (width 0.25) (layer B.Cu) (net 3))
 (segment (start 156.162267 74.610895) (end 156.162267 77.287145) (width 0.25) (layer B.Cu) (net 3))
 (segment (start 155.350599 78.098813) (end 155.0506 78.398812) (width 0.25) (layer B.Cu) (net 3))
 (via (at 155.0506 78.398812) (size 0.6) (drill 0.4) (layers F.Cu B.Cu) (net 3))
 (via (at 152.3976 81.2741) (size 0.6) (layers F.Cu B.Cu) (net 3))
 (segment (start 152.3917 81.28) (end 152.3976 81.2741) (width 0.25) (layer B.Cu) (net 3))
 (segment (start 151.13 81.28) (end 152.3917 81.28) (width 0.25) (layer B.Cu) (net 3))
 (segment (start 151.7904 76.962) (end 151.13 77.6224) (width 0.25) (layer B.Cu) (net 4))
 (segment (start 151.13 77.6224) (end 151.13 78.74) (width 0.25) (layer B.Cu) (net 4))
 (segment (start 155.1432 76.962) (end 151.7904 76.962) (width 0.25) (layer B.Cu) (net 4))
 (segment (start 155.5496 76.5556) (end 155.1432 76.962) (width 0.25) (layer B.Cu) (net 4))
 (segment (start 155.5496 75.0316) (end 155.5496 76.5556) (width 0.25) (layer B.Cu) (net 4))
 (segment (start 155.1305 74.6125) (end 155.5496 75.0316) (width 0.25) (layer B.Cu) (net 4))
 (segment (start 153.289 74.6125) (end 155.1305 74.6125) (width 0.25) (layer B.Cu) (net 4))
 (segment (start 153.289 74.6125) (end 153.664 74.6125) (width 0.25) (layer B.Cu) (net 4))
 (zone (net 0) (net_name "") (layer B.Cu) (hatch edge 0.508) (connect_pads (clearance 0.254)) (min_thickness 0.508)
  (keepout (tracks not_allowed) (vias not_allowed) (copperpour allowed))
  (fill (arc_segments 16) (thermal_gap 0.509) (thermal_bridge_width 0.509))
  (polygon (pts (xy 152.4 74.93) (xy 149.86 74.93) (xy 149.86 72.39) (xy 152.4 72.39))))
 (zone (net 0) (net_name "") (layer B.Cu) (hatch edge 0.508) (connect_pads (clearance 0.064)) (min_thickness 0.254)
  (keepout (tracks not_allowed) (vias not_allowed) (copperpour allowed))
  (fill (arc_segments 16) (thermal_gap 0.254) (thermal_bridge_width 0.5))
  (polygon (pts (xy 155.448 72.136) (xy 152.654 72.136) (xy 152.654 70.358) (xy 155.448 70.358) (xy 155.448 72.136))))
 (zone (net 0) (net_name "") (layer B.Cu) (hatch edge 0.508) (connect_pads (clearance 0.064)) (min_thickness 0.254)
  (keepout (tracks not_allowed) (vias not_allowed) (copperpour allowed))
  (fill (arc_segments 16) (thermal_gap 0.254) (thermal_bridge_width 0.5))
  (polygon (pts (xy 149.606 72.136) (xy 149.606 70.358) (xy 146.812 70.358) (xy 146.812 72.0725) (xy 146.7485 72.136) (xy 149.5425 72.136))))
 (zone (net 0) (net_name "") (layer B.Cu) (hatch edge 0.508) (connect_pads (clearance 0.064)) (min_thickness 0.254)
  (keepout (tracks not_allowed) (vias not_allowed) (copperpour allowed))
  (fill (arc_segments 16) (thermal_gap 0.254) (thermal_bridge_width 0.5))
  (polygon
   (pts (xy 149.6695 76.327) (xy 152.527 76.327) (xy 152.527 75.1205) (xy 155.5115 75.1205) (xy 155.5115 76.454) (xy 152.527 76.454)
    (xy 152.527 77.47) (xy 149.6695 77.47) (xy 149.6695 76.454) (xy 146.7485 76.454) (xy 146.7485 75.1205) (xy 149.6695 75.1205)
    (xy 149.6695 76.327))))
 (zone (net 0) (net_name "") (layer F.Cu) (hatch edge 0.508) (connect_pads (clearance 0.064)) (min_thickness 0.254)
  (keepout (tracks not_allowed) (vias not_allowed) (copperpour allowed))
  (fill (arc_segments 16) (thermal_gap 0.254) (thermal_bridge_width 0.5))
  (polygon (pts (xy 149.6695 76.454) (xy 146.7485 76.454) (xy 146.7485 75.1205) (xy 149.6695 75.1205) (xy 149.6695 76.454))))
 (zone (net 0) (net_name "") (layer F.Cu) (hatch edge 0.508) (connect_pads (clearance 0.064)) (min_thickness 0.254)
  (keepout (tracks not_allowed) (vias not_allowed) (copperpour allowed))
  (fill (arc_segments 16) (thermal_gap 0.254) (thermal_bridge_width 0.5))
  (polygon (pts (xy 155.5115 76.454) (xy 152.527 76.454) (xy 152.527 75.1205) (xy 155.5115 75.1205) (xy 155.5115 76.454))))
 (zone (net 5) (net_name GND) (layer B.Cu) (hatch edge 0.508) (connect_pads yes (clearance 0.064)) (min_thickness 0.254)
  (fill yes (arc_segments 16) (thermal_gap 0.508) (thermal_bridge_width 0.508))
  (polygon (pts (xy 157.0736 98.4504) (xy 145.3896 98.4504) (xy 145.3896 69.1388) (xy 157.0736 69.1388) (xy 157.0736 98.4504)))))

